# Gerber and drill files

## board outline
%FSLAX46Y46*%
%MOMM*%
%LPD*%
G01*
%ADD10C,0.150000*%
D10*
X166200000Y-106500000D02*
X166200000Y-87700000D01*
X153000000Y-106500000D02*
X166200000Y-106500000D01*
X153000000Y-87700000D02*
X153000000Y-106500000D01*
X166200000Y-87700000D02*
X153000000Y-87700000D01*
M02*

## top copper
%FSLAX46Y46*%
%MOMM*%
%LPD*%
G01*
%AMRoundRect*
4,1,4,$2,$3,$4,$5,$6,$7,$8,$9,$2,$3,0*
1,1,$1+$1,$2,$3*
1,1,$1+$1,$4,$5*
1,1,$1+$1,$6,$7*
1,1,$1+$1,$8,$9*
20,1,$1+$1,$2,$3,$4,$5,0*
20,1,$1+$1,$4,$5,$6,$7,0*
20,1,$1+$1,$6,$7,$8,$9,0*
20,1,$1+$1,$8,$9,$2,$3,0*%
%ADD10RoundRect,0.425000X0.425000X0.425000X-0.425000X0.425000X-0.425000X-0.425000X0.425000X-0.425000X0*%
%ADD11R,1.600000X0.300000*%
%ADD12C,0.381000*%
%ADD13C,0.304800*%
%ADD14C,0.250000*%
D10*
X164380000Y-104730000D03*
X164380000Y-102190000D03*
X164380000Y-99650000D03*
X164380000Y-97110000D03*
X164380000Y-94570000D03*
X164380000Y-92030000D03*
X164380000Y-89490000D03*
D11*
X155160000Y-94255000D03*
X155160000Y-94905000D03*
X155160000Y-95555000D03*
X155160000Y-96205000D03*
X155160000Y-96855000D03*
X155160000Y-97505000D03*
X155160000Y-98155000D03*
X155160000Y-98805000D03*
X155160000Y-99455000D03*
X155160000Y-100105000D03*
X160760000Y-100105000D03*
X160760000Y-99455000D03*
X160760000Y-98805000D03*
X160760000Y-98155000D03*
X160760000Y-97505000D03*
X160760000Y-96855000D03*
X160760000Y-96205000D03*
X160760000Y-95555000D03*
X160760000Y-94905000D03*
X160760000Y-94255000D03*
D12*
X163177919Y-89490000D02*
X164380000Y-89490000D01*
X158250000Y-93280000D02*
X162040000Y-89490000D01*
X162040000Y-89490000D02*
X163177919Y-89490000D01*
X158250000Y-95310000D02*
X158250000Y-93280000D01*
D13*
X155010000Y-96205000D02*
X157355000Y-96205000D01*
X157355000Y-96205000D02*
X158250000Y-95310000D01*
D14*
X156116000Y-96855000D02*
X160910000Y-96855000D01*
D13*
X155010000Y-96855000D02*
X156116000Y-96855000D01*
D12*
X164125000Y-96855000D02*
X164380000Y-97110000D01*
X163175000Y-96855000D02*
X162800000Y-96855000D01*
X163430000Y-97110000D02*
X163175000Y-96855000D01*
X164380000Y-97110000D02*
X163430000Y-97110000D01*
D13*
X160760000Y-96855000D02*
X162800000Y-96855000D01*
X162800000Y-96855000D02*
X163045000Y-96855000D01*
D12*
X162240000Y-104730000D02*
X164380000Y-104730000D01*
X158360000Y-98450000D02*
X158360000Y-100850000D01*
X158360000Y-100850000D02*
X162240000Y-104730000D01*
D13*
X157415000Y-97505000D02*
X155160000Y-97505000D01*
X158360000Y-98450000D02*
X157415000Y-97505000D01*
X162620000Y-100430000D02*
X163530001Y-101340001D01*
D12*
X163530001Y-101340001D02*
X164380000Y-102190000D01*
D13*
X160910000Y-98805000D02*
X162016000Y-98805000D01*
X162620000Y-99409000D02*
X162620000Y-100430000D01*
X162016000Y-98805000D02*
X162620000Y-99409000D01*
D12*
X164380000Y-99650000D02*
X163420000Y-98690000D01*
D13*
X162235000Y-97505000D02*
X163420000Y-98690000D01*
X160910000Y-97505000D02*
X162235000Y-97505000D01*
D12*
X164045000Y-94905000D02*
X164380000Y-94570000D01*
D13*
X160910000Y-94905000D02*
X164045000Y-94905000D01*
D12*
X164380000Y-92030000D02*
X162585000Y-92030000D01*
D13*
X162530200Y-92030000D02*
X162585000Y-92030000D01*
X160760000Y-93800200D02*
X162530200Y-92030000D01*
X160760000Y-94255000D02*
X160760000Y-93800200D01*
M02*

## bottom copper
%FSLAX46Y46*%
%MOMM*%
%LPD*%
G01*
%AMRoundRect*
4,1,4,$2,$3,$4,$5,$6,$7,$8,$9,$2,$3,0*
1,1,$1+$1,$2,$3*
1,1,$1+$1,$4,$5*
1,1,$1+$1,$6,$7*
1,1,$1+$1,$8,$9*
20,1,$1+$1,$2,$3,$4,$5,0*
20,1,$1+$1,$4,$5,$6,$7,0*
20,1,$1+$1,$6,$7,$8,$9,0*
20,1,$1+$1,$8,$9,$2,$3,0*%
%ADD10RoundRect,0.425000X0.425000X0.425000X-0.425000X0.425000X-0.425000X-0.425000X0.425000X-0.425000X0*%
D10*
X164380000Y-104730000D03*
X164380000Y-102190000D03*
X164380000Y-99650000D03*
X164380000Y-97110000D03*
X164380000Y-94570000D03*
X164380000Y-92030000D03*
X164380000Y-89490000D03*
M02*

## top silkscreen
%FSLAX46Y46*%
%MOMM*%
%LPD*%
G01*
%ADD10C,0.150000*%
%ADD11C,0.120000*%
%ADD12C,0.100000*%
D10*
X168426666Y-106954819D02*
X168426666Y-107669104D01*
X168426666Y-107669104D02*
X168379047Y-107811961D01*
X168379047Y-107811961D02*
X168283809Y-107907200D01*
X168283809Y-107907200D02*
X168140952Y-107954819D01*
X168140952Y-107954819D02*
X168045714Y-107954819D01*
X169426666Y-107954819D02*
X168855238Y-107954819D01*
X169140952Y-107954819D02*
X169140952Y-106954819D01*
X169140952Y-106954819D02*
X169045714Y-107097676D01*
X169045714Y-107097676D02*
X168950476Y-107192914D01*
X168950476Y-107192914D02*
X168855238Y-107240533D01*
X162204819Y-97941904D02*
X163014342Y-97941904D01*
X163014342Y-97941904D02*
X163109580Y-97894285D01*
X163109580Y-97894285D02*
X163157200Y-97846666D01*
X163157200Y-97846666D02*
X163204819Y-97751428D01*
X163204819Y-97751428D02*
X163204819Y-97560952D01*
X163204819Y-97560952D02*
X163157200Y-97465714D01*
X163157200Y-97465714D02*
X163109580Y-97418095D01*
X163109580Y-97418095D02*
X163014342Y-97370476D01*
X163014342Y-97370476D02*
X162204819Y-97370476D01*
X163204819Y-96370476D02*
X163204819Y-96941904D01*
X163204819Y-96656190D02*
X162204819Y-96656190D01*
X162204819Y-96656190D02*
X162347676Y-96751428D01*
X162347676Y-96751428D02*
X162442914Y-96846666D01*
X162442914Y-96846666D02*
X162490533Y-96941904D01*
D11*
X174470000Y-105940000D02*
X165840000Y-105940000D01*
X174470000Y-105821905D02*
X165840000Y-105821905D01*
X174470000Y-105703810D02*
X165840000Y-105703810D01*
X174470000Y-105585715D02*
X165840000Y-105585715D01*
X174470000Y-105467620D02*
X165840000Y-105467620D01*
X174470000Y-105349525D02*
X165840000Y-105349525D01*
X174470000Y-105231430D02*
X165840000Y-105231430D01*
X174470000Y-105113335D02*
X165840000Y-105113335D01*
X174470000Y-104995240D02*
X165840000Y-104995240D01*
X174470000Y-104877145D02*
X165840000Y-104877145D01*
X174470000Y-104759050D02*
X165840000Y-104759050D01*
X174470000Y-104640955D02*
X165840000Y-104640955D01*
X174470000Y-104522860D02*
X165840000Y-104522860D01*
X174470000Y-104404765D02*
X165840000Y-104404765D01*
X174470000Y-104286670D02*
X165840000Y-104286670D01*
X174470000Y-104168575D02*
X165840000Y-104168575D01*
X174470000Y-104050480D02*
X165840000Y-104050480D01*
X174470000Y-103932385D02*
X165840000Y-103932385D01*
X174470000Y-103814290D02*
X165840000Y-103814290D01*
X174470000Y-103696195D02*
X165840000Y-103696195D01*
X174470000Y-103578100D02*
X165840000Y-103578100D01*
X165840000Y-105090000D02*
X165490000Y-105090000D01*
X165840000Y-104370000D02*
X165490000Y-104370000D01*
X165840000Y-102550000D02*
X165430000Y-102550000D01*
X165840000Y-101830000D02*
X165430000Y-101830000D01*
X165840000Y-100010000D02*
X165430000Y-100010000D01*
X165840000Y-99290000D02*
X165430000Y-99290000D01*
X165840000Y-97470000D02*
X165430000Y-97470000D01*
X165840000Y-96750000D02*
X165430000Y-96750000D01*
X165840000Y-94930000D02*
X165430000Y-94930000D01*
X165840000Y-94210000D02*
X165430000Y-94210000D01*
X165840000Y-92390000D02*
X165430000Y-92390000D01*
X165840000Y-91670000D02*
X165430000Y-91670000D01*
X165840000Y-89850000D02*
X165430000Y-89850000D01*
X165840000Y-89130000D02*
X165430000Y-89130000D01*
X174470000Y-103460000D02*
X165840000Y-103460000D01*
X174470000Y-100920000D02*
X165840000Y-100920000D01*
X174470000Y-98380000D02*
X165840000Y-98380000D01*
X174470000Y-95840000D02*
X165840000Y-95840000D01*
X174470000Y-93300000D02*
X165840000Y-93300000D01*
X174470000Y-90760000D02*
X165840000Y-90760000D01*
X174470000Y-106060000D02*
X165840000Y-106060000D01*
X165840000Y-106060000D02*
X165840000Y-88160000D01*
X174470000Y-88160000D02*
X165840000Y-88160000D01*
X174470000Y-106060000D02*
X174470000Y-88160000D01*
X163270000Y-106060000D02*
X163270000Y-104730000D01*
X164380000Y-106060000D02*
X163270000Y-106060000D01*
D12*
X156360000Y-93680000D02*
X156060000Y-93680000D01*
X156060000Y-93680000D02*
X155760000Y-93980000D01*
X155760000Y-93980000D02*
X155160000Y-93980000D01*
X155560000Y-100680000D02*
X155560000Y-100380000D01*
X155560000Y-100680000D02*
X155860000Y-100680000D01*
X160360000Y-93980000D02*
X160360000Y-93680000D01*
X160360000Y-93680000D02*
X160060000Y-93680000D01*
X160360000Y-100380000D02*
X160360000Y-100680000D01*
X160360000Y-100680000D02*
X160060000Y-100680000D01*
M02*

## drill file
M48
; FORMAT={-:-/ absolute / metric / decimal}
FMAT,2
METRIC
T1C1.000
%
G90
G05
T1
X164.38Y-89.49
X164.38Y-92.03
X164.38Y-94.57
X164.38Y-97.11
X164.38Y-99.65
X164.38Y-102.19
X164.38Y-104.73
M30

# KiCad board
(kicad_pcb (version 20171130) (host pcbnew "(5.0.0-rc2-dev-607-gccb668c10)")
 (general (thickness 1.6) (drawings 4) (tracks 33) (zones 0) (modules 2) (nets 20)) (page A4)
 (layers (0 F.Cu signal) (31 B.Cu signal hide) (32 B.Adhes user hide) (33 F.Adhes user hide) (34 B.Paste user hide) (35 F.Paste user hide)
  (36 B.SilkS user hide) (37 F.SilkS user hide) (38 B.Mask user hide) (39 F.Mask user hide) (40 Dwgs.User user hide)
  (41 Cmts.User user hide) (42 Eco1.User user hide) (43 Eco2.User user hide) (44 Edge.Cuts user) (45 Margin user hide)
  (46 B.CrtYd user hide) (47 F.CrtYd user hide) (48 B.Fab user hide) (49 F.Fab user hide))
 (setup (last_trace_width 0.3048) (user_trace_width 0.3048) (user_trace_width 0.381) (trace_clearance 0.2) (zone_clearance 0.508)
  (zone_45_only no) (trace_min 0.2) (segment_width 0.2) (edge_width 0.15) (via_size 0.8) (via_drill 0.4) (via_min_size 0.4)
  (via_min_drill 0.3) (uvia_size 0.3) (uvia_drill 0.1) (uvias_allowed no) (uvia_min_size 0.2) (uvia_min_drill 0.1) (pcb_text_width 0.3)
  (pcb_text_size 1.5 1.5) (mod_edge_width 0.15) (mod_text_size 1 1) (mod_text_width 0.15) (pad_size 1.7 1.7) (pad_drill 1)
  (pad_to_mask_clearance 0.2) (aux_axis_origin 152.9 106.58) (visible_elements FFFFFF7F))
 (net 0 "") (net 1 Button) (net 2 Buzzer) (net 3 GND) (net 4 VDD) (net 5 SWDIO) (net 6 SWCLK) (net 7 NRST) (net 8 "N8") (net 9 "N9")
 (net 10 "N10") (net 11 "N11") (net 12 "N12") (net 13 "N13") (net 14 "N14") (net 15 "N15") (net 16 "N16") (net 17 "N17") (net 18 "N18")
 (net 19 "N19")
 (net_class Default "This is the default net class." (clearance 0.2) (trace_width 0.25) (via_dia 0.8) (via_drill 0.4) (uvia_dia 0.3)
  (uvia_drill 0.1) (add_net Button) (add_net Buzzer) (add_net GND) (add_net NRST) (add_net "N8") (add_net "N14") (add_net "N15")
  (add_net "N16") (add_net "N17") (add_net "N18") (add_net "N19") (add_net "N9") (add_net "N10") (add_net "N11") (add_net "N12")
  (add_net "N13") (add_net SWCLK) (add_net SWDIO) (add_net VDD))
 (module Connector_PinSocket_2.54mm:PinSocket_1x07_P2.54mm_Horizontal (layer F.Cu) (at 164.38 104.73 180)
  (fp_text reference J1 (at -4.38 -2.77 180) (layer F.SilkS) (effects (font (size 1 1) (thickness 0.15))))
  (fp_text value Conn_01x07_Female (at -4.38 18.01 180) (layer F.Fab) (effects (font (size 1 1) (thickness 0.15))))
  (fp_line (start -10.09 -1.21) (end -1.46 -1.21) (layer F.SilkS) (width 0.12))
  (fp_line (start -10.09 -1.091905) (end -1.46 -1.091905) (layer F.SilkS) (width 0.12))
  (fp_line (start -10.09 -0.97381) (end -1.46 -0.97381) (layer F.SilkS) (width 0.12))
  (fp_line (start -10.09 -0.855715) (end -1.46 -0.855715) (layer F.SilkS) (width 0.12))
  (fp_line (start -10.09 -0.73762) (end -1.46 -0.73762) (layer F.SilkS) (width 0.12))
  (fp_line (start -10.09 -0.619525) (end -1.46 -0.619525) (layer F.SilkS) (width 0.12))
  (fp_line (start -10.09 -0.50143) (end -1.46 -0.50143) (layer F.SilkS) (width 0.12))
  (fp_line (start -10.09 -0.383335) (end -1.46 -0.383335) (layer F.SilkS) (width 0.12))
  (fp_line (start -10.09 -0.26524) (end -1.46 -0.26524) (layer F.SilkS) (width 0.12))
  (fp_line (start -10.09 -0.147145) (end -1.46 -0.147145) (layer F.SilkS) (width 0.12))
  (fp_line (start -10.09 -0.02905) (end -1.46 -0.02905) (layer F.SilkS) (width 0.12))
  (fp_line (start -10.09 0.089045) (end -1.46 0.089045) (layer F.SilkS) (width 0.12))
  (fp_line (start -10.09 0.20714) (end -1.46 0.20714) (layer F.SilkS) (width 0.12))
  (fp_line (start -10.09 0.325235) (end -1.46 0.325235) (layer F.SilkS) (width 0.12))
  (fp_line (start -10.09 0.44333) (end -1.46 0.44333) (layer F.SilkS) (width 0.12))
  (fp_line (start -10.09 0.561425) (end -1.46 0.561425) (layer F.SilkS) (width 0.12))
  (fp_line (start -10.09 0.67952) (end -1.46 0.67952) (layer F.SilkS) (width 0.12))
  (fp_line (start -10.09 0.797615) (end -1.46 0.797615) (layer F.SilkS) (width 0.12))
  (fp_line (start -10.09 0.91571) (end -1.46 0.91571) (layer F.SilkS) (width 0.12))
  (fp_line (start -10.09 1.033805) (end -1.46 1.033805) (layer F.SilkS) (width 0.12))
  (fp_line (start -10.09 1.1519) (end -1.46 1.1519) (layer F.SilkS) (width 0.12))
  (fp_line (start -1.46 -0.36) (end -1.11 -0.36) (layer F.SilkS) (width 0.12))
  (fp_line (start -1.46 0.36) (end -1.11 0.36) (layer F.SilkS) (width 0.12))
  (fp_line (start -1.46 2.18) (end -1.05 2.18) (layer F.SilkS) (width 0.12))
  (fp_line (start -1.46 2.9) (end -1.05 2.9) (layer F.SilkS) (width 0.12))
  (fp_line (start -1.46 4.72) (end -1.05 4.72) (layer F.SilkS) (width 0.12))
  (fp_line (start -1.46 5.44) (end -1.05 5.44) (layer F.SilkS) (width 0.12))
  (fp_line (start -1.46 7.26) (end -1.05 7.26) (layer F.SilkS) (width 0.12))
  (fp_line (start -1.46 7.98) (end -1.05 7.98) (layer F.SilkS) (width 0.12))
  (fp_line (start -1.46 9.8) (end -1.05 9.8) (layer F.SilkS) (width 0.12))
  (fp_line (start -1.46 10.52) (end -1.05 10.52) (layer F.SilkS) (width 0.12))
  (fp_line (start -1.46 12.34) (end -1.05 12.34) (layer F.SilkS) (width 0.12))
  (fp_line (start -1.46 13.06) (end -1.05 13.06) (layer F.SilkS) (width 0.12))
  (fp_line (start -1.46 14.88) (end -1.05 14.88) (layer F.SilkS) (width 0.12))
  (fp_line (start -1.46 15.6) (end -1.05 15.6) (layer F.SilkS) (width 0.12))
  (fp_line (start -10.09 1.27) (end -1.46 1.27) (layer F.SilkS) (width 0.12))
  (fp_line (start -10.09 3.81) (end -1.46 3.81) (layer F.SilkS) (width 0.12))
  (fp_line (start -10.09 6.35) (end -1.46 6.35) (layer F.SilkS) (width 0.12))
  (fp_line (start -10.09 8.89) (end -1.46 8.89) (layer F.SilkS) (width 0.12))
  (fp_line (start -10.09 11.43) (end -1.46 11.43) (layer F.SilkS) (width 0.12))
  (fp_line (start -10.09 13.97) (end -1.46 13.97) (layer F.SilkS) (width 0.12))
  (fp_line (start -10.09 -1.33) (end -1.46 -1.33) (layer F.SilkS) (width 0.12))
  (fp_line (start -1.46 -1.33) (end -1.46 16.57) (layer F.SilkS) (width 0.12))
  (fp_line (start -10.09 16.57) (end -1.46 16.57) (layer F.SilkS) (width 0.12))
  (fp_line (start -10.09 -1.33) (end -10.09 16.57) (layer F.SilkS) (width 0.12))
  (fp_line (start 1.11 -1.33) (end 1.11 0) (layer F.SilkS) (width 0.12))
  (fp_line (start 0 -1.33) (end 1.11 -1.33) (layer F.SilkS) (width 0.12))
  (pad 1 thru_hole roundrect (at 0 0 180) (size 1.7 1.7) (drill 1) (layers *.Cu *.Mask) (roundrect_rratio 0.25) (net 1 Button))
  (pad 2 thru_hole roundrect (at 0 2.54 180) (size 1.7 1.7) (drill 1) (layers *.Cu *.Mask) (roundrect_rratio 0.25) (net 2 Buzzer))
  (pad 3 thru_hole roundrect (at 0 5.08 180) (size 1.7 1.7) (drill 1) (layers *.Cu *.Mask) (roundrect_rratio 0.25) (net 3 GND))
  (pad 4 thru_hole roundrect (at 0 7.62 180) (size 1.7 1.7) (drill 1) (layers *.Cu *.Mask) (roundrect_rratio 0.25) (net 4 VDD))
  (pad 5 thru_hole roundrect (at 0 10.16 180) (size 1.7 1.7) (drill 1) (layers *.Cu *.Mask) (roundrect_rratio 0.25) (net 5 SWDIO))
  (pad 6 thru_hole roundrect (at 0 12.7 180) (size 1.7 1.7) (drill 1) (layers *.Cu *.Mask) (roundrect_rratio 0.25) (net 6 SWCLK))
  (pad 7 thru_hole roundrect (at 0 15.24 180) (size 1.7 1.7) (drill 1) (layers *.Cu *.Mask) (roundrect_rratio 0.25) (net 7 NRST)))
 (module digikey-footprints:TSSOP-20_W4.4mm (layer F.Cu) (at 157.96 97.18 270)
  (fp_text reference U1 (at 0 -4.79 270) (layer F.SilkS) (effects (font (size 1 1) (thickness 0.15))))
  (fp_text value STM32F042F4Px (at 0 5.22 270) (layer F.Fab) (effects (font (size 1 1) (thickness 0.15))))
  (fp_line (start -3.5 1.6) (end -3.5 1.9) (layer F.SilkS) (width 0.1))
  (fp_line (start -3.5 1.9) (end -3.2 2.2) (layer F.SilkS) (width 0.1))
  (fp_line (start -3.2 2.2) (end -3.2 2.8) (layer F.SilkS) (width 0.1))
  (fp_line (start 3.5 2.4) (end 3.2 2.4) (layer F.SilkS) (width 0.1))
  (fp_line (start 3.5 2.4) (end 3.5 2.1) (layer F.SilkS) (width 0.1))
  (fp_line (start -3.2 -2.4) (end -3.5 -2.4) (layer F.SilkS) (width 0.1))
  (fp_line (start -3.5 -2.4) (end -3.5 -2.1) (layer F.SilkS) (width 0.1))
  (fp_line (start 3.2 -2.4) (end 3.5 -2.4) (layer F.SilkS) (width 0.1))
  (fp_line (start 3.5 -2.4) (end 3.5 -2.1) (layer F.SilkS) (width 0.1))
  (pad 1 smd rect (at -2.925 2.8 270) (size 0.3 1.6) (layers F.Cu F.Paste F.Mask) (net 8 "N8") (solder_mask_margin 0.07))
  (pad 2 smd rect (at -2.275 2.8 270) (size 0.3 1.6) (layers F.Cu F.Paste F.Mask) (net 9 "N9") (solder_mask_margin 0.07))
  (pad 3 smd rect (at -1.625 2.8 270) (size 0.3 1.6) (layers F.Cu F.Paste F.Mask) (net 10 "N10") (solder_mask_margin 0.07))
  (pad 4 smd rect (at -0.975 2.8 270) (size 0.3 1.6) (layers F.Cu F.Paste F.Mask) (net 7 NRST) (solder_mask_margin 0.07))
  (pad 5 smd rect (at -0.325 2.8 270) (size 0.3 1.6) (layers F.Cu F.Paste F.Mask) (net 4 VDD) (solder_mask_margin 0.07))
  (pad 6 smd rect (at 0.325 2.8 270) (size 0.3 1.6) (layers F.Cu F.Paste F.Mask) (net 1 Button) (solder_mask_margin 0.07))
  (pad 7 smd rect (at 0.975 2.8 270) (size 0.3 1.6) (layers F.Cu F.Paste F.Mask) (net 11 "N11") (solder_mask_margin 0.07))
  (pad 8 smd rect (at 1.625 2.8 270) (size 0.3 1.6) (layers F.Cu F.Paste F.Mask) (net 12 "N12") (solder_mask_margin 0.07))
  (pad 9 smd rect (at 2.275 2.8 270) (size 0.3 1.6) (layers F.Cu F.Paste F.Mask) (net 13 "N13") (solder_mask_margin 0.07))
  (pad 10 smd rect (at 2.925 2.8 270) (size 0.3 1.6) (layers F.Cu F.Paste F.Mask) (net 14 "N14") (solder_mask_margin 0.07))
  (pad 11 smd rect (at 2.925 -2.8 270) (size 0.3 1.6) (layers F.Cu F.Paste F.Mask) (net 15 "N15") (solder_mask_margin 0.07))
  (pad 12 smd rect (at 2.275 -2.8 270) (size 0.3 1.6) (layers F.Cu F.Paste F.Mask) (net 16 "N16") (solder_mask_margin 0.07))
  (pad 13 smd rect (at 1.625 -2.8 270) (size 0.3 1.6) (layers F.Cu F.Paste F.Mask) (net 2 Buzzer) (solder_mask_margin 0.07))
  (pad 14 smd rect (at 0.975 -2.8 270) (size 0.3 1.6) (layers F.Cu F.Paste F.Mask) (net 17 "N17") (solder_mask_margin 0.07))
  (pad 15 smd rect (at 0.325 -2.8 270) (size 0.3 1.6) (layers F.Cu F.Paste F.Mask) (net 3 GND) (solder_mask_margin 0.07))
  (pad 16 smd rect (at -0.325 -2.8 270) (size 0.3 1.6) (layers F.Cu F.Paste F.Mask) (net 4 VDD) (solder_mask_margin 0.07))
  (pad 17 smd rect (at -0.975 -2.8 270) (size 0.3 1.6) (layers F.Cu F.Paste F.Mask) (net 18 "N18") (solder_mask_margin 0.07))
  (pad 18 smd rect (at -1.625 -2.8 270) (size 0.3 1.6) (layers F.Cu F.Paste F.Mask) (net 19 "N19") (solder_mask_margin 0.07))
  (pad 19 smd rect (at -2.275 -2.8 270) (size 0.3 1.6) (layers F.Cu F.Paste F.Mask) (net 5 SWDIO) (solder_mask_margin 0.07))
  (pad 20 smd rect (at -2.925 -2.8 270) (size 0.3 1.6) (layers F.Cu F.Paste F.Mask) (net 6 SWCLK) (solder_mask_margin 0.07)))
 (gr_line (start 166.2 106.5) (end 166.2 87.7) (layer Edge.Cuts) (width 0.15))
 (gr_line (start 153 106.5) (end 166.2 106.5) (layer Edge.Cuts) (width 0.15))
 (gr_line (start 153 87.7) (end 153 106.5) (layer Edge.Cuts) (width 0.15))
 (gr_line (start 166.2 87.7) (end 153 87.7) (layer Edge.Cuts) (width 0.15))
 (segment (start 163.177919 89.49) (end 164.38 89.49) (width 0.381) (layer F.Cu) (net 7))
 (segment (start 158.25 93.28) (end 162.04 89.49) (width 0.381) (layer F.Cu) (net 7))
 (segment (start 162.04 89.49) (end 163.177919 89.49) (width 0.381) (layer F.Cu) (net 7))
 (segment (start 158.25 95.31) (end 158.25 93.28) (width 0.381) (layer F.Cu) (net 7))
 (segment (start 155.01 96.205) (end 157.355 96.205) (width 0.3048) (layer F.Cu) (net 7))
 (segment (start 157.355 96.205) (end 158.25 95.31) (width 0.3048) (layer F.Cu) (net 7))
 (segment (start 156.116 96.855) (end 160.91 96.855) (width 0.25) (layer F.Cu) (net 4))
 (segment (start 155.01 96.855) (end 156.116 96.855) (width 0.3048) (layer F.Cu) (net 4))
 (segment (start 164.125 96.855) (end 164.38 97.11) (width 0.381) (layer F.Cu) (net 4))
 (segment (start 163.175 96.855) (end 162.8 96.855) (width 0.381) (layer F.Cu) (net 4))
 (segment (start 163.43 97.11) (end 163.175 96.855) (width 0.381) (layer F.Cu) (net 4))
 (segment (start 164.38 97.11) (end 163.43 97.11) (width 0.381) (layer F.Cu) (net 4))
 (segment (start 160.76 96.855) (end 162.8 96.855) (width 0.3048) (layer F.Cu) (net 4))
 (segment (start 162.8 96.855) (end 163.045 96.855) (width 0.3048) (layer F.Cu) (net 4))
 (segment (start 162.24 104.73) (end 164.38 104.73) (width 0.381) (layer F.Cu) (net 1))
 (segment (start 158.36 98.45) (end 158.36 100.85) (width 0.381) (layer F.Cu) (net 1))
 (segment (start 158.36 100.85) (end 162.24 104.73) (width 0.381) (layer F.Cu) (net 1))
 (segment (start 157.415 97.505) (end 155.16 97.505) (width 0.3048) (layer F.Cu) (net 1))
 (segment (start 158.36 98.45) (end 157.415 97.505) (width 0.3048) (layer F.Cu) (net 1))
 (segment (start 162.62 100.43) (end 163.530001 101.340001) (width 0.3048) (layer F.Cu) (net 2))
 (segment (start 163.530001 101.340001) (end 164.38 102.19) (width 0.381) (layer F.Cu) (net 2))
 (segment (start 160.91 98.805) (end 162.016 98.805) (width 0.3048) (layer F.Cu) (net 2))
 (segment (start 162.62 99.409) (end 162.62 100.43) (width 0.3048) (layer F.Cu) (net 2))
 (segment (start 162.016 98.805) (end 162.62 99.409) (width 0.3048) (layer F.Cu) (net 2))
 (segment (start 164.38 99.65) (end 163.42 98.69) (width 0.381) (layer F.Cu) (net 3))
 (segment (start 162.235 97.505) (end 163.42 98.69) (width 0.3048) (layer F.Cu) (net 3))
 (segment (start 160.91 97.505) (end 162.235 97.505) (width 0.3048) (layer F.Cu) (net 3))
 (segment (start 164.045 94.905) (end 164.38 94.57) (width 0.381) (layer F.Cu) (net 5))
 (segment (start 160.91 94.905) (end 164.045 94.905) (width 0.3048) (layer F.Cu) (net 5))
 (segment (start 164.38 92.03) (end 162.585 92.03) (width 0.381) (layer F.Cu) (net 6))
 (segment (start 162.5302 92.03) (end 162.585 92.03) (width 0.3048) (layer F.Cu) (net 6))
 (segment (start 160.76 93.8002) (end 162.5302 92.03) (width 0.3048) (layer F.Cu) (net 6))
 (segment (start 160.76 94.255) (end 160.76 93.8002) (width 0.3048) (layer F.Cu) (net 6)))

